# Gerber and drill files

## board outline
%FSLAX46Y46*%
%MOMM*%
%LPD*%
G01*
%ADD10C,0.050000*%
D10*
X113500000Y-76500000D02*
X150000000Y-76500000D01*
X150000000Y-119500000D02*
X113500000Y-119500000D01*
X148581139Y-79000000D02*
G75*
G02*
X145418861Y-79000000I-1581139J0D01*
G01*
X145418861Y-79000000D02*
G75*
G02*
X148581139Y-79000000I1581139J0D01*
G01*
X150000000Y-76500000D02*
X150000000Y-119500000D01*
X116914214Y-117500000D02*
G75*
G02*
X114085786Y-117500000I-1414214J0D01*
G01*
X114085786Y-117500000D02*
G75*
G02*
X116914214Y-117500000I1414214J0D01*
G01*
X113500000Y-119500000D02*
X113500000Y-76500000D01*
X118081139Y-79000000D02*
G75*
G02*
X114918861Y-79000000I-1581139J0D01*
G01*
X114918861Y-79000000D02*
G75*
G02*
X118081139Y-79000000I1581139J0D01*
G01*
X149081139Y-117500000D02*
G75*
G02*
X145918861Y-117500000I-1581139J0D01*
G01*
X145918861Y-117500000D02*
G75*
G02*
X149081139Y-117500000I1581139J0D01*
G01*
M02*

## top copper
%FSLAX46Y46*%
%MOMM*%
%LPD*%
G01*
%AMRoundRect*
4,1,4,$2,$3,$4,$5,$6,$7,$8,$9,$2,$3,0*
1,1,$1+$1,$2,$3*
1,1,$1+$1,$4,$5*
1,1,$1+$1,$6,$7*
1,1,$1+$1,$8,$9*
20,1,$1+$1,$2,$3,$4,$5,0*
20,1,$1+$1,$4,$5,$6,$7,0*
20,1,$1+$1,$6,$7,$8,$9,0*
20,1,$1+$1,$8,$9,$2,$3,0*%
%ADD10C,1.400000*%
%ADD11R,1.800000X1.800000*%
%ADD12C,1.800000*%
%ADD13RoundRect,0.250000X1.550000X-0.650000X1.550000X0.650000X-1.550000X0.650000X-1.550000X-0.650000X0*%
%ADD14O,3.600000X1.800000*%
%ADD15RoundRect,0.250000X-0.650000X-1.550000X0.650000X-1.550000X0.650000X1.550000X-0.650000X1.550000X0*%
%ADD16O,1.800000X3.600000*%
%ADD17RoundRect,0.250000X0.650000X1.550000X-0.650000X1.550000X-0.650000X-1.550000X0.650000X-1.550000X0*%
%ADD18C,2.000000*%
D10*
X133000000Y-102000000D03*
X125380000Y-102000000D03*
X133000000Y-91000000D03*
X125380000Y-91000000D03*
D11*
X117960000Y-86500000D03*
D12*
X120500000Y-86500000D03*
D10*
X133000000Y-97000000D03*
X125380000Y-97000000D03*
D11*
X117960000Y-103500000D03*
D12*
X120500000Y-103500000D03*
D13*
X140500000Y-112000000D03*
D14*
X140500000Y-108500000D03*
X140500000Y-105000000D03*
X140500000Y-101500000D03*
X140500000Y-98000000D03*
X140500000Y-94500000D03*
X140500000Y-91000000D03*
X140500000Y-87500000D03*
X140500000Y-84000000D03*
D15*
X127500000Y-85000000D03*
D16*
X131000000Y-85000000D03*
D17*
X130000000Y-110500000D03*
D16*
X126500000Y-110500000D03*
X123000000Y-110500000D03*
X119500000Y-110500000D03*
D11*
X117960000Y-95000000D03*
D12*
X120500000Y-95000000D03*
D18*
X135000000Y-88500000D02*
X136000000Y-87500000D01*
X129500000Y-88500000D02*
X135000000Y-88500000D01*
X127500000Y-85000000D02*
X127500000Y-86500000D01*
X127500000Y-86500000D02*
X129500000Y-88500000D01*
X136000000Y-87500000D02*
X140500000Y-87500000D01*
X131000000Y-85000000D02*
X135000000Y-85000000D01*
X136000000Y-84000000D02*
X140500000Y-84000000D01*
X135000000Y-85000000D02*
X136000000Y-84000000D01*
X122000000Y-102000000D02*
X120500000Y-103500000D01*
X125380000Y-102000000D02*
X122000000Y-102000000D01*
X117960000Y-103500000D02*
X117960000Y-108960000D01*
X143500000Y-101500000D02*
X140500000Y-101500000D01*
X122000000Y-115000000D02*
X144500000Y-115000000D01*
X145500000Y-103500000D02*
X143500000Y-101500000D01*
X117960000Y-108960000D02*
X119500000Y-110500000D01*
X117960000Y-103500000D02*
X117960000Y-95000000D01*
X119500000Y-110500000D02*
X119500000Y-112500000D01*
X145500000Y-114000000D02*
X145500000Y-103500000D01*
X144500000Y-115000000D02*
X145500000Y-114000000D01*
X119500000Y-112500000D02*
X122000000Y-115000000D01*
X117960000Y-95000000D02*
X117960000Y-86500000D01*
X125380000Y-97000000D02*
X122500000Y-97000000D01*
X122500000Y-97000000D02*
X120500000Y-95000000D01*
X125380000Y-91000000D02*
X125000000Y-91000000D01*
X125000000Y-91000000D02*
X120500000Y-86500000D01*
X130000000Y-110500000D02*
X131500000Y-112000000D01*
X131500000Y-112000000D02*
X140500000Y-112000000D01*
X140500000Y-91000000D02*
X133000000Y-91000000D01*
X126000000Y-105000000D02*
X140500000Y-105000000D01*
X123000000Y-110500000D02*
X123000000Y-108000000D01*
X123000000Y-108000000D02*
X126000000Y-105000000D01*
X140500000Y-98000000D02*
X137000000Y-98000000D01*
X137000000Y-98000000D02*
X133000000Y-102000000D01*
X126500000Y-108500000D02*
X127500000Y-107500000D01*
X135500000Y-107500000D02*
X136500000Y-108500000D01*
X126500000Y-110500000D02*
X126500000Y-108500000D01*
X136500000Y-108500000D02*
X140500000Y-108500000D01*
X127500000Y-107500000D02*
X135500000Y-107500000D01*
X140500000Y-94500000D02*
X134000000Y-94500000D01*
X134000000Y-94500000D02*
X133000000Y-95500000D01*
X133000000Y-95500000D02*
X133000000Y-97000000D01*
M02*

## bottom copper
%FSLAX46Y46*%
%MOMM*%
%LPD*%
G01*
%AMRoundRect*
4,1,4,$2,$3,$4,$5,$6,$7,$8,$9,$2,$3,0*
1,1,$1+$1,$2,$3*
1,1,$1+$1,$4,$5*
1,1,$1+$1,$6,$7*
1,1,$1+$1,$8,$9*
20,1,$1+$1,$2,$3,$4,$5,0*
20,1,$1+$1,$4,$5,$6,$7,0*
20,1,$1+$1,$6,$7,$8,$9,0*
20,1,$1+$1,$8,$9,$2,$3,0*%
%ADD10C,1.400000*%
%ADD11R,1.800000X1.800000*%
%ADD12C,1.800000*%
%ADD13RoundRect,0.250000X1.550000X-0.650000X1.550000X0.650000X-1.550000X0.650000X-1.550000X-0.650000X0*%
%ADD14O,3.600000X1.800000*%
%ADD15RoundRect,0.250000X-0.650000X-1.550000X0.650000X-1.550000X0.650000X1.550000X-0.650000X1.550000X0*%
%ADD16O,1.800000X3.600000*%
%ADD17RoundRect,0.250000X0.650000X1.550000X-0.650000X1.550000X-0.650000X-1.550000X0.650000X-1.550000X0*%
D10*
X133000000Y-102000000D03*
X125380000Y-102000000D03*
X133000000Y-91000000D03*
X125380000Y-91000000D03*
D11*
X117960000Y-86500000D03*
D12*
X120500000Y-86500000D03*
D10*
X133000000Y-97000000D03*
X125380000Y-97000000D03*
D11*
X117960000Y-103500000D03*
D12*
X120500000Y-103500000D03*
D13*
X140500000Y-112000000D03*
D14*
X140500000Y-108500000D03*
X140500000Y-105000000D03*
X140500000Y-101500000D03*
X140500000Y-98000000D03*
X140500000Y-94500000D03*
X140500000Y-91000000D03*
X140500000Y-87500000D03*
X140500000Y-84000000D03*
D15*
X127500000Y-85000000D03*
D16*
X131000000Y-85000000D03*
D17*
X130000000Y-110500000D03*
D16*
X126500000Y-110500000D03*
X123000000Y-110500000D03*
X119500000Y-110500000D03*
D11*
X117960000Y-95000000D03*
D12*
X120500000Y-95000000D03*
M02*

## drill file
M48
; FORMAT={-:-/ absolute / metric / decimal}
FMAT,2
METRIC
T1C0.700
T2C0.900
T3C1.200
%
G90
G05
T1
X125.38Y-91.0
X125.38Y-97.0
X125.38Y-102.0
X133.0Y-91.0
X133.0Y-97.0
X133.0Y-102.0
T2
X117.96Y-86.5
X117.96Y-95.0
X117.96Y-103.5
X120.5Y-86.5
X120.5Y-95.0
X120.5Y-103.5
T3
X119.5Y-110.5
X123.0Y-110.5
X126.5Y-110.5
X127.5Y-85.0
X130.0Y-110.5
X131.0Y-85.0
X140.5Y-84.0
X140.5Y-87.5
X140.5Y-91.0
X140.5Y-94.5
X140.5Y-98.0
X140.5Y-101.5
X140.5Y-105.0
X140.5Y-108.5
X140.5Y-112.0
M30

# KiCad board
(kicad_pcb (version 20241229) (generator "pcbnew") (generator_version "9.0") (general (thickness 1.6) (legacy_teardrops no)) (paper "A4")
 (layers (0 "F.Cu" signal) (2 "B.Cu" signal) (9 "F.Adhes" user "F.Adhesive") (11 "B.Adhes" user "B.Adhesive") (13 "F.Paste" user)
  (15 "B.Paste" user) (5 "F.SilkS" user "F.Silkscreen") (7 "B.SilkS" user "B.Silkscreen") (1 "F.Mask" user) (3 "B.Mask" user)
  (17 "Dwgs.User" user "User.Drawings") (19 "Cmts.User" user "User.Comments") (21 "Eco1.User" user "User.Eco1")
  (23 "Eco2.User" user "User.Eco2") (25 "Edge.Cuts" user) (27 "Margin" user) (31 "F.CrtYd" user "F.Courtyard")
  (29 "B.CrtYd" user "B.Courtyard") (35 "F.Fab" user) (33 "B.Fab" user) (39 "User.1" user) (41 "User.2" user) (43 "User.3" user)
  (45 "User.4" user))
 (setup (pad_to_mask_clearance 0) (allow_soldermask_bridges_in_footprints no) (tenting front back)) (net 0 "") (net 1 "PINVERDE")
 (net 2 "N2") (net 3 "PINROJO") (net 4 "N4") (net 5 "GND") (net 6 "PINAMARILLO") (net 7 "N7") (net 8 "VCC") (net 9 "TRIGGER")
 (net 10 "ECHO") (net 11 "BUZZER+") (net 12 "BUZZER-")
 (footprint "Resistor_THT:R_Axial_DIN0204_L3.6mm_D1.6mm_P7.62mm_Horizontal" (layer "F.Cu") (at 133 102 180)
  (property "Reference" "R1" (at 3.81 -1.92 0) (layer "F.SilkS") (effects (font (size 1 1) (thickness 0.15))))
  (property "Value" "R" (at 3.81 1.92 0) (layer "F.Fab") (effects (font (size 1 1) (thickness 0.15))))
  (pad "1" thru_hole circle (at 0 0 180) (size 1.4 1.4) (drill 0.7) (layers "*.Cu" "*.Mask") (remove_unused_layers no) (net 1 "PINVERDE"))
  (pad "2" thru_hole circle (at 7.62 0 180) (size 1.4 1.4) (drill 0.7) (layers "*.Cu" "*.Mask") (remove_unused_layers no) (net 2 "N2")))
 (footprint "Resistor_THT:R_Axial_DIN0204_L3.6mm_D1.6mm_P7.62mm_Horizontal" (layer "F.Cu") (at 133 91 180)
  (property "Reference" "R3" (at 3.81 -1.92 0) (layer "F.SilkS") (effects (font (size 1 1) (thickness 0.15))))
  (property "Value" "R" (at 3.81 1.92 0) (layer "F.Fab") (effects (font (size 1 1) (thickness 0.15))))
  (pad "1" thru_hole circle (at 0 0 180) (size 1.4 1.4) (drill 0.7) (layers "*.Cu" "*.Mask") (remove_unused_layers no) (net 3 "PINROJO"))
  (pad "2" thru_hole circle (at 7.62 0 180) (size 1.4 1.4) (drill 0.7) (layers "*.Cu" "*.Mask") (remove_unused_layers no) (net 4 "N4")))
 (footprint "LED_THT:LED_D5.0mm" (layer "F.Cu") (at 117.96 86.5)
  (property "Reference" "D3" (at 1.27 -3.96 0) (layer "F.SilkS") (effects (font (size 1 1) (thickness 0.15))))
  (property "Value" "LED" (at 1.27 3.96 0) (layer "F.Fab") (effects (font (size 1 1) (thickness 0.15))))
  (pad "1" thru_hole rect (at 0 0) (size 1.8 1.8) (drill 0.9) (layers "*.Cu" "*.Mask") (remove_unused_layers no) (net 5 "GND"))
  (pad "2" thru_hole circle (at 2.54 0) (size 1.8 1.8) (drill 0.9) (layers "*.Cu" "*.Mask") (remove_unused_layers no) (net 4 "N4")))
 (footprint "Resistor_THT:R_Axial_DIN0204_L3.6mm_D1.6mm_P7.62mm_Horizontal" (layer "F.Cu") (at 133 97 180)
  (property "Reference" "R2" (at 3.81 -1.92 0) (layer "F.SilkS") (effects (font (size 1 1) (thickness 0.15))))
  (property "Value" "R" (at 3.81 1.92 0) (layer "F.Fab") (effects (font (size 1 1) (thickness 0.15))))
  (pad "1" thru_hole circle (at 0 0 180) (size 1.4 1.4) (drill 0.7) (layers "*.Cu" "*.Mask") (remove_unused_layers no) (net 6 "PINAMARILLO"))
  (pad "2" thru_hole circle (at 7.62 0 180) (size 1.4 1.4) (drill 0.7) (layers "*.Cu" "*.Mask") (remove_unused_layers no) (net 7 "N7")))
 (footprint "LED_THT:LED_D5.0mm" (layer "F.Cu") (at 117.96 103.5)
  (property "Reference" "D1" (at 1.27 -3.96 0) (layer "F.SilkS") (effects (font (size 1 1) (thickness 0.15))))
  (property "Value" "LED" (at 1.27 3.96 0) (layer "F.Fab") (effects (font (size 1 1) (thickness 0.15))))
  (pad "1" thru_hole rect (at 0 0) (size 1.8 1.8) (drill 0.9) (layers "*.Cu" "*.Mask") (remove_unused_layers no) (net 5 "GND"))
  (pad "2" thru_hole circle (at 2.54 0) (size 1.8 1.8) (drill 0.9) (layers "*.Cu" "*.Mask") (remove_unused_layers no) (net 2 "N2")))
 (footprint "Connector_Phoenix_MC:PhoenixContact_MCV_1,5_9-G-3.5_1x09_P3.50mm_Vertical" (layer "F.Cu") (at 140.5 112 90)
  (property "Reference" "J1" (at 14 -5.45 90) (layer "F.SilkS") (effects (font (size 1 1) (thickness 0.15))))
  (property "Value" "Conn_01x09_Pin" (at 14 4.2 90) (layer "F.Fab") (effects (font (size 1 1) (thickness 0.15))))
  (pad "1" thru_hole roundrect (at 0 0 90) (size 1.8 3.6) (drill 1.2) (layers "*.Cu" "*.Mask") (remove_unused_layers no)
   (roundrect_rratio 0.138889) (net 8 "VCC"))
  (pad "2" thru_hole oval (at 3.5 0 90) (size 1.8 3.6) (drill 1.2) (layers "*.Cu" "*.Mask") (remove_unused_layers no) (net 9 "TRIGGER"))
  (pad "3" thru_hole oval (at 7 0 90) (size 1.8 3.6) (drill 1.2) (layers "*.Cu" "*.Mask") (remove_unused_layers no) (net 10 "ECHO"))
  (pad "4" thru_hole oval (at 10.5 0 90) (size 1.8 3.6) (drill 1.2) (layers "*.Cu" "*.Mask") (remove_unused_layers no) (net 5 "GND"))
  (pad "5" thru_hole oval (at 14 0 90) (size 1.8 3.6) (drill 1.2) (layers "*.Cu" "*.Mask") (remove_unused_layers no) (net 1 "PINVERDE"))
  (pad "6" thru_hole oval (at 17.5 0 90) (size 1.8 3.6) (drill 1.2) (layers "*.Cu" "*.Mask") (remove_unused_layers no) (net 6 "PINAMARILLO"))
  (pad "7" thru_hole oval (at 21 0 90) (size 1.8 3.6) (drill 1.2) (layers "*.Cu" "*.Mask") (remove_unused_layers no) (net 3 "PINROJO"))
  (pad "8" thru_hole oval (at 24.5 0 90) (size 1.8 3.6) (drill 1.2) (layers "*.Cu" "*.Mask") (remove_unused_layers no) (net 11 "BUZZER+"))
  (pad "9" thru_hole oval (at 28 0 90) (size 1.8 3.6) (drill 1.2) (layers "*.Cu" "*.Mask") (remove_unused_layers no) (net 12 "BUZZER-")))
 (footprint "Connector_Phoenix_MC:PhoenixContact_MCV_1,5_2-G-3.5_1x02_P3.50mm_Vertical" (layer "F.Cu") (at 127.5 85)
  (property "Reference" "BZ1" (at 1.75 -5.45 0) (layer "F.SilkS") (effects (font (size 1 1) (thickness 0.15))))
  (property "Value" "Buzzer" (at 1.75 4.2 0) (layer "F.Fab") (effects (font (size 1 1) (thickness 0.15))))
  (pad "1" thru_hole roundrect (at 0 0) (size 1.8 3.6) (drill 1.2) (layers "*.Cu" "*.Mask") (remove_unused_layers no)
   (roundrect_rratio 0.138889) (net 11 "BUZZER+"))
  (pad "2" thru_hole oval (at 3.5 0) (size 1.8 3.6) (drill 1.2) (layers "*.Cu" "*.Mask") (remove_unused_layers no) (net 12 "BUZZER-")))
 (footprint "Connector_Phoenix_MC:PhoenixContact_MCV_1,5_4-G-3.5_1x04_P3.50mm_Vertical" (layer "F.Cu") (at 130 110.5 180)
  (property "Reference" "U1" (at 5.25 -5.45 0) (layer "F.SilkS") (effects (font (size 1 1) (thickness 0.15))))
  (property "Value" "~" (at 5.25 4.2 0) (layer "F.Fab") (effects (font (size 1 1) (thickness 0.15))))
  (pad "1" thru_hole roundrect (at 0 0 180) (size 1.8 3.6) (drill 1.2) (layers "*.Cu" "*.Mask") (remove_unused_layers no)
   (roundrect_rratio 0.138889) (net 8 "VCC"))
  (pad "2" thru_hole oval (at 3.5 0 180) (size 1.8 3.6) (drill 1.2) (layers "*.Cu" "*.Mask") (remove_unused_layers no) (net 9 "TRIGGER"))
  (pad "3" thru_hole oval (at 7 0 180) (size 1.8 3.6) (drill 1.2) (layers "*.Cu" "*.Mask") (remove_unused_layers no) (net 10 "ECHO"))
  (pad "4" thru_hole oval (at 10.5 0 180) (size 1.8 3.6) (drill 1.2) (layers "*.Cu" "*.Mask") (remove_unused_layers no) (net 5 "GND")))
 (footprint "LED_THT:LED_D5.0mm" (layer "F.Cu") (at 117.96 95)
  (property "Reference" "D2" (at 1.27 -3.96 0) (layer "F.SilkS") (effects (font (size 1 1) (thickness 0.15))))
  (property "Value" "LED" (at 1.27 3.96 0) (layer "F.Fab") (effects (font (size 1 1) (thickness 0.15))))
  (pad "1" thru_hole rect (at 0 0) (size 1.8 1.8) (drill 0.9) (layers "*.Cu" "*.Mask") (remove_unused_layers no) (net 5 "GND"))
  (pad "2" thru_hole circle (at 2.54 0) (size 1.8 1.8) (drill 0.9) (layers "*.Cu" "*.Mask") (remove_unused_layers no) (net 7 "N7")))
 (gr_line (start 113.5 76.5) (end 150 76.5) (stroke (width 0.05) (type default)) (layer "Edge.Cuts"))
 (gr_line (start 150 119.5) (end 113.5 119.5) (stroke (width 0.05) (type default)) (layer "Edge.Cuts"))
 (gr_circle (center 147 79) (end 147.5 77.5) (stroke (width 0.05) (type default)) (fill no) (layer "Edge.Cuts"))
 (gr_line (start 150 76.5) (end 150 119.5) (stroke (width 0.05) (type default)) (layer "Edge.Cuts"))
 (gr_circle (center 115.5 117.5) (end 116.5 116.5) (stroke (width 0.05) (type default)) (fill no) (layer "Edge.Cuts"))
 (gr_line (start 113.5 119.5) (end 113.5 76.5) (stroke (width 0.05) (type default)) (layer "Edge.Cuts"))
 (gr_circle (center 116.5 79) (end 118 79.5) (stroke (width 0.05) (type default)) (fill no) (layer "Edge.Cuts"))
 (gr_circle (center 147.5 117.5) (end 148 116) (stroke (width 0.05) (type default)) (fill no) (layer "Edge.Cuts"))
 (segment (start 135 88.5) (end 136 87.5) (width 2) (layer "F.Cu") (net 11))
 (segment (start 129.5 88.5) (end 135 88.5) (width 2) (layer "F.Cu") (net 11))
 (segment (start 127.5 85) (end 127.5 86.5) (width 2) (layer "F.Cu") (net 11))
 (segment (start 127.5 86.5) (end 129.5 88.5) (width 2) (layer "F.Cu") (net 11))
 (segment (start 136 87.5) (end 140.5 87.5) (width 2) (layer "F.Cu") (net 11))
 (segment (start 131 85) (end 135 85) (width 2) (layer "F.Cu") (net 12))
 (segment (start 136 84) (end 140.5 84) (width 2) (layer "F.Cu") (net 12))
 (segment (start 135 85) (end 136 84) (width 2) (layer "F.Cu") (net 12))
 (segment (start 122 102) (end 120.5 103.5) (width 2) (layer "F.Cu") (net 2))
 (segment (start 125.38 102) (end 122 102) (width 2) (layer "F.Cu") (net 2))
 (segment (start 117.96 103.5) (end 117.96 108.96) (width 2) (layer "F.Cu") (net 5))
 (segment (start 143.5 101.5) (end 140.5 101.5) (width 2) (layer "F.Cu") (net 5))
 (segment (start 122 115) (end 144.5 115) (width 2) (layer "F.Cu") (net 5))
 (segment (start 145.5 103.5) (end 143.5 101.5) (width 2) (layer "F.Cu") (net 5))
 (segment (start 117.96 108.96) (end 119.5 110.5) (width 2) (layer "F.Cu") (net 5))
 (segment (start 117.96 103.5) (end 117.96 95) (width 2) (layer "F.Cu") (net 5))
 (segment (start 119.5 110.5) (end 119.5 112.5) (width 2) (layer "F.Cu") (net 5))
 (segment (start 145.5 114) (end 145.5 103.5) (width 2) (layer "F.Cu") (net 5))
 (segment (start 144.5 115) (end 145.5 114) (width 2) (layer "F.Cu") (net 5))
 (segment (start 119.5 112.5) (end 122 115) (width 2) (layer "F.Cu") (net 5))
 (segment (start 117.96 95) (end 117.96 86.5) (width 2) (layer "F.Cu") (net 5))
 (segment (start 125.38 97) (end 122.5 97) (width 2) (layer "F.Cu") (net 7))
 (segment (start 122.5 97) (end 120.5 95) (width 2) (layer "F.Cu") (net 7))
 (segment (start 125.38 91) (end 125 91) (width 2) (layer "F.Cu") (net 4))
 (segment (start 125 91) (end 120.5 86.5) (width 2) (layer "F.Cu") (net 4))
 (segment (start 130 110.5) (end 131.5 112) (width 2) (layer "F.Cu") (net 8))
 (segment (start 131.5 112) (end 140.5 112) (width 2) (layer "F.Cu") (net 8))
 (segment (start 140.5 91) (end 133 91) (width 2) (layer "F.Cu") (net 3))
 (segment (start 126 105) (end 140.5 105) (width 2) (layer "F.Cu") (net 10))
 (segment (start 123 110.5) (end 123 108) (width 2) (layer "F.Cu") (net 10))
 (segment (start 123 108) (end 126 105) (width 2) (layer "F.Cu") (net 10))
 (segment (start 140.5 98) (end 137 98) (width 2) (layer "F.Cu") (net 1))
 (segment (start 137 98) (end 133 102) (width 2) (layer "F.Cu") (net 1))
 (segment (start 126.5 108.5) (end 127.5 107.5) (width 2) (layer "F.Cu") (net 9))
 (segment (start 135.5 107.5) (end 136.5 108.5) (width 2) (layer "F.Cu") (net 9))
 (segment (start 126.5 110.5) (end 126.5 108.5) (width 2) (layer "F.Cu") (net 9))
 (segment (start 136.5 108.5) (end 140.5 108.5) (width 2) (layer "F.Cu") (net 9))
 (segment (start 127.5 107.5) (end 135.5 107.5) (width 2) (layer "F.Cu") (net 9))
 (segment (start 140.5 94.5) (end 134 94.5) (width 2) (layer "F.Cu") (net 6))
 (segment (start 134 94.5) (end 133 95.5) (width 2) (layer "F.Cu") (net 6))
 (segment (start 133 95.5) (end 133 97) (width 2) (layer "F.Cu") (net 6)))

